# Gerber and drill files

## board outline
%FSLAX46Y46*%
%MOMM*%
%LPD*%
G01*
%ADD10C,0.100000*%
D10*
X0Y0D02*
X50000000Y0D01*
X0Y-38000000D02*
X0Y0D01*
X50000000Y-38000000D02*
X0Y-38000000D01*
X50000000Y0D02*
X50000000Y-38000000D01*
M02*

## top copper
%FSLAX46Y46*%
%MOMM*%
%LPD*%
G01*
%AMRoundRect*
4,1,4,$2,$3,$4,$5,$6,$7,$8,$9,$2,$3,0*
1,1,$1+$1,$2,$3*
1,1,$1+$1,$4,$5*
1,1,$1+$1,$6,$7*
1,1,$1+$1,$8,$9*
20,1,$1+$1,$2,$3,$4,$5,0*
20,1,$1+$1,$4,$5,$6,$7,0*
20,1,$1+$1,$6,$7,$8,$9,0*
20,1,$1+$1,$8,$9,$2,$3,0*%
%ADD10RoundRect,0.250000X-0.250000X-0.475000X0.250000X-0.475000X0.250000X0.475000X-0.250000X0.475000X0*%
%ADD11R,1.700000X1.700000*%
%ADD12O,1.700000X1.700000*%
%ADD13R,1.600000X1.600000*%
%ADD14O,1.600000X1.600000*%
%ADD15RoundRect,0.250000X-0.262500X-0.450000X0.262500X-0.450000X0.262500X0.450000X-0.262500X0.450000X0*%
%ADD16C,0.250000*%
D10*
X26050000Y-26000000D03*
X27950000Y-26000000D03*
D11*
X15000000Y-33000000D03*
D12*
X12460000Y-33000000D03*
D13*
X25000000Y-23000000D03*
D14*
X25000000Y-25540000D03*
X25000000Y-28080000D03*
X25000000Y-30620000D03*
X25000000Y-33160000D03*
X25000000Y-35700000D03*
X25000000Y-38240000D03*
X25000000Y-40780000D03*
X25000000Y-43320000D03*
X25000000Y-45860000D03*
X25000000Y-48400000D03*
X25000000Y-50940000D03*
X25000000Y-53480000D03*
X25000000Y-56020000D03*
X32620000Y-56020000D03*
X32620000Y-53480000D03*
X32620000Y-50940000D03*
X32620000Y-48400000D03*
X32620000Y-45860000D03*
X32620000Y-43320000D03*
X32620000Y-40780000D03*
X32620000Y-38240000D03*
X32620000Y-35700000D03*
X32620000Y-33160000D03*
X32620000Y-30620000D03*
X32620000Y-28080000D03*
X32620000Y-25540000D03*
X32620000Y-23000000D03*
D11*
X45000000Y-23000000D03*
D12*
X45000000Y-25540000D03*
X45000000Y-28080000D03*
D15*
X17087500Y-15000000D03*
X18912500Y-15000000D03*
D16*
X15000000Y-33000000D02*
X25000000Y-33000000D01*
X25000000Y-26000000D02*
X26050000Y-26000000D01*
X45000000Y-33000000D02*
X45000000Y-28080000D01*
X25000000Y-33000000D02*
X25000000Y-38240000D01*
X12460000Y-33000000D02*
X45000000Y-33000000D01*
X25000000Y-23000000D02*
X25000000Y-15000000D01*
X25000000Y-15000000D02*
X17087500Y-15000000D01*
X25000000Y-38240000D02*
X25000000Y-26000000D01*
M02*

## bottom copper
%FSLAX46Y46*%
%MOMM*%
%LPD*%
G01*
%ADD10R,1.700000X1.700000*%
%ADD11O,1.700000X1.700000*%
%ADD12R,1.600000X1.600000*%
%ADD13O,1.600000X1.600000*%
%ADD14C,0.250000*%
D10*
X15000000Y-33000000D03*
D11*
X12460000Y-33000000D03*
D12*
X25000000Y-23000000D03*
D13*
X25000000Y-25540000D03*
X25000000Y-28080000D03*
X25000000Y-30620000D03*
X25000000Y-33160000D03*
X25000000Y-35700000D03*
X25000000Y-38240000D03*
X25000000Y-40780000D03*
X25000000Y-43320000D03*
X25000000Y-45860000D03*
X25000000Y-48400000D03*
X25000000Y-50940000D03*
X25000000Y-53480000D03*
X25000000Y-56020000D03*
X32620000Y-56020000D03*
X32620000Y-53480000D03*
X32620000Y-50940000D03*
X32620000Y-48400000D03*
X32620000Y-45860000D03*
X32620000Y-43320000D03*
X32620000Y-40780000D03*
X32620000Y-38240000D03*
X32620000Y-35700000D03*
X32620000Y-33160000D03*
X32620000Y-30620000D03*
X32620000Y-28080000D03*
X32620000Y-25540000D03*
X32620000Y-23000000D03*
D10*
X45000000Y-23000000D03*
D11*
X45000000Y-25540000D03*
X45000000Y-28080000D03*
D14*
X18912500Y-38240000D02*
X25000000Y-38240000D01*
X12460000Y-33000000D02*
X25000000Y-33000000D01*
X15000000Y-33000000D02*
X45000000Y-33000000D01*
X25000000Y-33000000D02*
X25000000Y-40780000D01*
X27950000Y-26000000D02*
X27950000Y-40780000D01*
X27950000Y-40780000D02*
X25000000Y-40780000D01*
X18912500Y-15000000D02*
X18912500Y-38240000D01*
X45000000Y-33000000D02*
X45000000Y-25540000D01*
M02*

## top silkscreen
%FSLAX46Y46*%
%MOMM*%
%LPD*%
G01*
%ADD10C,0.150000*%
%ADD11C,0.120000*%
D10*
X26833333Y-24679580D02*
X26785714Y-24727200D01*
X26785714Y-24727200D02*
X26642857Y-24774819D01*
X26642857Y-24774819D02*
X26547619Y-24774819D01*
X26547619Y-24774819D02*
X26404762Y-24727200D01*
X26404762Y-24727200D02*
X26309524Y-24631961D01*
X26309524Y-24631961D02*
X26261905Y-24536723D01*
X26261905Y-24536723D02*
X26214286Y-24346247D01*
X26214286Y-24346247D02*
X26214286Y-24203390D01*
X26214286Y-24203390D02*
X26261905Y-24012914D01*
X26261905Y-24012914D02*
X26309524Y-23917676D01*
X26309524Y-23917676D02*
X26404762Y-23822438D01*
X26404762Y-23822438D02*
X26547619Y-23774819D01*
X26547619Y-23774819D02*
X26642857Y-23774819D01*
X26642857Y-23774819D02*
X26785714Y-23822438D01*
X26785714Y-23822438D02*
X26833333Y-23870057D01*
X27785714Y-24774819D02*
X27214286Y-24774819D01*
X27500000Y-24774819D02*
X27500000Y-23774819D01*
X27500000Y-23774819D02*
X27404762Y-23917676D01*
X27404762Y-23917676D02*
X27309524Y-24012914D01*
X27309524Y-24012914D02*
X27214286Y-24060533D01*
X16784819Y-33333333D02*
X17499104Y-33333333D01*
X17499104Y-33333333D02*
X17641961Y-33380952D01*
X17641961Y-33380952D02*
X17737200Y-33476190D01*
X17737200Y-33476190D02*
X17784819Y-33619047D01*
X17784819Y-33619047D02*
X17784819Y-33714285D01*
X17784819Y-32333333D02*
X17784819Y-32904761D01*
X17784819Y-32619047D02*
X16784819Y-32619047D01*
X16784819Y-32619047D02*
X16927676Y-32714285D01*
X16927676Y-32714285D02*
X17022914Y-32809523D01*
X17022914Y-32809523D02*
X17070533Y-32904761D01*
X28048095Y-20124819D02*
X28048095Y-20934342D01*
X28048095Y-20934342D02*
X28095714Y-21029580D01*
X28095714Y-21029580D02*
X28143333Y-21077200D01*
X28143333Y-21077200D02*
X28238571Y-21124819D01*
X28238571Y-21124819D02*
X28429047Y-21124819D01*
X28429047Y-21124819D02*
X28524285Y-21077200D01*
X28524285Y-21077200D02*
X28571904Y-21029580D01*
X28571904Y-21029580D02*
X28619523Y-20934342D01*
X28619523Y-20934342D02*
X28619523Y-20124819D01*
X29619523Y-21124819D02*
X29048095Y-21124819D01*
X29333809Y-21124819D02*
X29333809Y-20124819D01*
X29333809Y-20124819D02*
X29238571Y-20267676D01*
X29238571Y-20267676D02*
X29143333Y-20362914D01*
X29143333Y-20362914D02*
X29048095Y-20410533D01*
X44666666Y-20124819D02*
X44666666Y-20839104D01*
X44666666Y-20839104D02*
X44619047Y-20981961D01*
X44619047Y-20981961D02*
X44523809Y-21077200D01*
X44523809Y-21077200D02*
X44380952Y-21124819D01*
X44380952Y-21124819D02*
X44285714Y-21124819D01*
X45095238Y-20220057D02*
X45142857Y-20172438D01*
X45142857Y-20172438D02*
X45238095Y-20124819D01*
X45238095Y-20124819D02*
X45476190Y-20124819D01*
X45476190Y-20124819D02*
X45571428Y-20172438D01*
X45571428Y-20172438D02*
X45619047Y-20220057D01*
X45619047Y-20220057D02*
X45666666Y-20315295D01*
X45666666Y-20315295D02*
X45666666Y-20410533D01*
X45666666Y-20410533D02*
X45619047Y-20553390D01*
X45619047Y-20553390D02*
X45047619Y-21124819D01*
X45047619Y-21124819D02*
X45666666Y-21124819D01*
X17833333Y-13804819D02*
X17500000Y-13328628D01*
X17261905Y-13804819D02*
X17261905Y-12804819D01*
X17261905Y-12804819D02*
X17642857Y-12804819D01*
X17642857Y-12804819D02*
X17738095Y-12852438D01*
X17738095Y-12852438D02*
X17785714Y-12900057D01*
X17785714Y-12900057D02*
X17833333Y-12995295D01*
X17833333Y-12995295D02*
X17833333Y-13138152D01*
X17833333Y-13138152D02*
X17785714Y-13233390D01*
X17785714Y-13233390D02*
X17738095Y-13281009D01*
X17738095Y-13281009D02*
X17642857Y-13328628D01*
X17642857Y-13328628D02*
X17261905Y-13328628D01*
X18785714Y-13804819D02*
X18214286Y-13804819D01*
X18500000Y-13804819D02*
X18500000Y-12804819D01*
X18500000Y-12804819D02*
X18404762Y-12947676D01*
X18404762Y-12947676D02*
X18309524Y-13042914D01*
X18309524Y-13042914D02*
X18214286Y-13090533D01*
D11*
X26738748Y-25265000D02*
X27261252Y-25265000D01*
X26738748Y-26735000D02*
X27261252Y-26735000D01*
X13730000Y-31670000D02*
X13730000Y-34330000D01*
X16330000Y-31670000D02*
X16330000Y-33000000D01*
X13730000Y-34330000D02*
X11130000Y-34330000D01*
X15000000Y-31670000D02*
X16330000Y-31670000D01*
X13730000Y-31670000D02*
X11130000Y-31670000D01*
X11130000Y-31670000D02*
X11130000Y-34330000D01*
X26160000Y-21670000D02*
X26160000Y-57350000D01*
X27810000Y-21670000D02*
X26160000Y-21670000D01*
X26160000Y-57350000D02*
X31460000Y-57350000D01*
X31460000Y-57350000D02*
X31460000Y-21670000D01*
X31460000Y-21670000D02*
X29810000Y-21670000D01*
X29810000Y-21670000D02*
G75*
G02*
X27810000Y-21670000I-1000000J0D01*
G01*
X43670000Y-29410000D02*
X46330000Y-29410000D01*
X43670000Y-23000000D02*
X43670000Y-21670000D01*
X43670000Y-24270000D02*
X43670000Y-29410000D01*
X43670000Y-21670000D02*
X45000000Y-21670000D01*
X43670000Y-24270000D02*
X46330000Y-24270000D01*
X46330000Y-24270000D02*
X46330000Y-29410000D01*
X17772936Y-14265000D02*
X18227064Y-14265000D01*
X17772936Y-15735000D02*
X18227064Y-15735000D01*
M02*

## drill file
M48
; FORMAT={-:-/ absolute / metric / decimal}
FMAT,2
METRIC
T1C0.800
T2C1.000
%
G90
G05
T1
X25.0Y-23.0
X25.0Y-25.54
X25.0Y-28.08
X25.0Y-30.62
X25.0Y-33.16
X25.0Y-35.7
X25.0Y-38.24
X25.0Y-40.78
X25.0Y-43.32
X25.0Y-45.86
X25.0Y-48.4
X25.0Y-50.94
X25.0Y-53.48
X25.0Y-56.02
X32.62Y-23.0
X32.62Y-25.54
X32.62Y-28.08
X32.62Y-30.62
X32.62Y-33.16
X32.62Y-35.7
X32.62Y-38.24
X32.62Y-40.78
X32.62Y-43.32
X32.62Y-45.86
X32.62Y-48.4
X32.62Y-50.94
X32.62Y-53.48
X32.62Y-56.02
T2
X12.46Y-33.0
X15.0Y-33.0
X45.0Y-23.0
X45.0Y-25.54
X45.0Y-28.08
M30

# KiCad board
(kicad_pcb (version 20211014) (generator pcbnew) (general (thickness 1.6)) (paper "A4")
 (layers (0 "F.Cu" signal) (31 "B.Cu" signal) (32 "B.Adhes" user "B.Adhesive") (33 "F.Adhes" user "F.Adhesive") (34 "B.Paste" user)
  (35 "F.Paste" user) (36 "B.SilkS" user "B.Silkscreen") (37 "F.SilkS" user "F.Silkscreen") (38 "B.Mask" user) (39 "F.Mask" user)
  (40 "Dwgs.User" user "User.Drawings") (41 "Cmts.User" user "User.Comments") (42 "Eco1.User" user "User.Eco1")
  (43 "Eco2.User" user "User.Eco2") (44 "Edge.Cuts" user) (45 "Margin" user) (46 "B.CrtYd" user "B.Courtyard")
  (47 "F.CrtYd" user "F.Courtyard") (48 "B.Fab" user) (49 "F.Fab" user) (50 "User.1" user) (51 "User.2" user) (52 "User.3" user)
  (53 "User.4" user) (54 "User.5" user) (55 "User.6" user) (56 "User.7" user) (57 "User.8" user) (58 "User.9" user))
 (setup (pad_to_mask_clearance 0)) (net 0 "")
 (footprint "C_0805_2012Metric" (layer "F.Cu") (at 27 26)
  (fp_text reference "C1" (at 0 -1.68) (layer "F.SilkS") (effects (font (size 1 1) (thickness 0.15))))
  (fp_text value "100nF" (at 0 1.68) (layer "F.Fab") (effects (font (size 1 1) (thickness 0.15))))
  (fp_line (start -0.261252 -0.735) (end 0.261252 -0.735) (layer "F.SilkS") (width 0.12))
  (fp_line (start -0.261252 0.735) (end 0.261252 0.735) (layer "F.SilkS") (width 0.12))
  (pad "1" smd roundrect (at -0.95 0) (size 1 1.45) (layers "F.Cu" "F.Paste" "F.Mask") (roundrect_rratio 0.25))
  (pad "2" smd roundrect (at 0.95 0) (size 1 1.45) (layers "F.Cu" "F.Paste" "F.Mask") (roundrect_rratio 0.25)))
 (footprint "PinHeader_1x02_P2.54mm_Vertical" (layer "F.Cu") (at 15 33 -90)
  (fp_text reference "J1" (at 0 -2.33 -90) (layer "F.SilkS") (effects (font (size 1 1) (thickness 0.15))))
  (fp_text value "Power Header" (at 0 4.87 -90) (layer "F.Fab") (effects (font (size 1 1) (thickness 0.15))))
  (fp_line (start -1.33 1.27) (end 1.33 1.27) (layer "F.SilkS") (width 0.12))
  (fp_line (start -1.33 -1.33) (end 0 -1.33) (layer "F.SilkS") (width 0.12))
  (fp_line (start 1.33 1.27) (end 1.33 3.87) (layer "F.SilkS") (width 0.12))
  (fp_line (start -1.33 0) (end -1.33 -1.33) (layer "F.SilkS") (width 0.12))
  (fp_line (start -1.33 1.27) (end -1.33 3.87) (layer "F.SilkS") (width 0.12))
  (fp_line (start -1.33 3.87) (end 1.33 3.87) (layer "F.SilkS") (width 0.12))
  (pad "1" thru_hole rect (at 0 0 270) (size 1.7 1.7) (drill 1) (layers *.Cu *.Mask))
  (pad "2" thru_hole oval (at 0 2.54 270) (size 1.7 1.7) (drill 1) (layers *.Cu *.Mask)))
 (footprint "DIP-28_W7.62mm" (layer "F.Cu") (at 25 23)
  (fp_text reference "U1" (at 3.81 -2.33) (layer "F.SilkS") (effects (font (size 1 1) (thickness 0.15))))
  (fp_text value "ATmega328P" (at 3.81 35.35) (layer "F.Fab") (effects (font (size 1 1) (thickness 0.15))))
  (fp_line (start 1.16 -1.33) (end 1.16 34.35) (layer "F.SilkS") (width 0.12))
  (fp_line (start 2.81 -1.33) (end 1.16 -1.33) (layer "F.SilkS") (width 0.12))
  (fp_line (start 1.16 34.35) (end 6.46 34.35) (layer "F.SilkS") (width 0.12))
  (fp_line (start 6.46 34.35) (end 6.46 -1.33) (layer "F.SilkS") (width 0.12))
  (fp_line (start 6.46 -1.33) (end 4.81 -1.33) (layer "F.SilkS") (width 0.12))
  (fp_arc (start 4.81 -1.33) (mid 3.81 -0.33) (end 2.81 -1.33) (layer "F.SilkS") (width 0.12))
  (pad "1" thru_hole rect (at 0 0) (size 1.6 1.6) (drill 0.8) (layers *.Cu *.Mask))
  (pad "2" thru_hole oval (at 0 2.54) (size 1.6 1.6) (drill 0.8) (layers *.Cu *.Mask))
  (pad "3" thru_hole oval (at 0 5.08) (size 1.6 1.6) (drill 0.8) (layers *.Cu *.Mask))
  (pad "4" thru_hole oval (at 0 7.62) (size 1.6 1.6) (drill 0.8) (layers *.Cu *.Mask))
  (pad "5" thru_hole oval (at 0 10.16) (size 1.6 1.6) (drill 0.8) (layers *.Cu *.Mask))
  (pad "6" thru_hole oval (at 0 12.7) (size 1.6 1.6) (drill 0.8) (layers *.Cu *.Mask))
  (pad "7" thru_hole oval (at 0 15.24) (size 1.6 1.6) (drill 0.8) (layers *.Cu *.Mask))
  (pad "8" thru_hole oval (at 0 17.78) (size 1.6 1.6) (drill 0.8) (layers *.Cu *.Mask))
  (pad "9" thru_hole oval (at 0 20.32) (size 1.6 1.6) (drill 0.8) (layers *.Cu *.Mask))
  (pad "10" thru_hole oval (at 0 22.86) (size 1.6 1.6) (drill 0.8) (layers *.Cu *.Mask))
  (pad "11" thru_hole oval (at 0 25.4) (size 1.6 1.6) (drill 0.8) (layers *.Cu *.Mask))
  (pad "12" thru_hole oval (at 0 27.94) (size 1.6 1.6) (drill 0.8) (layers *.Cu *.Mask))
  (pad "13" thru_hole oval (at 0 30.48) (size 1.6 1.6) (drill 0.8) (layers *.Cu *.Mask))
  (pad "14" thru_hole oval (at 0 33.02) (size 1.6 1.6) (drill 0.8) (layers *.Cu *.Mask))
  (pad "15" thru_hole oval (at 7.62 33.02) (size 1.6 1.6) (drill 0.8) (layers *.Cu *.Mask))
  (pad "16" thru_hole oval (at 7.62 30.48) (size 1.6 1.6) (drill 0.8) (layers *.Cu *.Mask))
  (pad "17" thru_hole oval (at 7.62 27.94) (size 1.6 1.6) (drill 0.8) (layers *.Cu *.Mask))
  (pad "18" thru_hole oval (at 7.62 25.4) (size 1.6 1.6) (drill 0.8) (layers *.Cu *.Mask))
  (pad "19" thru_hole oval (at 7.62 22.86) (size 1.6 1.6) (drill 0.8) (layers *.Cu *.Mask))
  (pad "20" thru_hole oval (at 7.62 20.32) (size 1.6 1.6) (drill 0.8) (layers *.Cu *.Mask))
  (pad "21" thru_hole oval (at 7.62 17.78) (size 1.6 1.6) (drill 0.8) (layers *.Cu *.Mask))
  (pad "22" thru_hole oval (at 7.62 15.24) (size 1.6 1.6) (drill 0.8) (layers *.Cu *.Mask))
  (pad "23" thru_hole oval (at 7.62 12.7) (size 1.6 1.6) (drill 0.8) (layers *.Cu *.Mask))
  (pad "24" thru_hole oval (at 7.62 10.16) (size 1.6 1.6) (drill 0.8) (layers *.Cu *.Mask))
  (pad "25" thru_hole oval (at 7.62 7.62) (size 1.6 1.6) (drill 0.8) (layers *.Cu *.Mask))
  (pad "26" thru_hole oval (at 7.62 5.08) (size 1.6 1.6) (drill 0.8) (layers *.Cu *.Mask))
  (pad "27" thru_hole oval (at 7.62 2.54) (size 1.6 1.6) (drill 0.8) (layers *.Cu *.Mask))
  (pad "28" thru_hole oval (at 7.62 0) (size 1.6 1.6) (drill 0.8) (layers *.Cu *.Mask)))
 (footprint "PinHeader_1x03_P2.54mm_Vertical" (layer "F.Cu") (at 45 23)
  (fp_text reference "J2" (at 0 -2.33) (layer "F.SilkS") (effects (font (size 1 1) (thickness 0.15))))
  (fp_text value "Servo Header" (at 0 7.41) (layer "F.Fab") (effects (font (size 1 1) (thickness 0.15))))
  (fp_line (start -1.33 6.41) (end 1.33 6.41) (layer "F.SilkS") (width 0.12))
  (fp_line (start -1.33 0) (end -1.33 -1.33) (layer "F.SilkS") (width 0.12))
  (fp_line (start -1.33 1.27) (end -1.33 6.41) (layer "F.SilkS") (width 0.12))
  (fp_line (start -1.33 -1.33) (end 0 -1.33) (layer "F.SilkS") (width 0.12))
  (fp_line (start -1.33 1.27) (end 1.33 1.27) (layer "F.SilkS") (width 0.12))
  (fp_line (start 1.33 1.27) (end 1.33 6.41) (layer "F.SilkS") (width 0.12))
  (pad "1" thru_hole rect (at 0 0) (size 1.7 1.7) (drill 1) (layers *.Cu *.Mask))
  (pad "2" thru_hole oval (at 0 2.54) (size 1.7 1.7) (drill 1) (layers *.Cu *.Mask))
  (pad "3" thru_hole oval (at 0 5.08) (size 1.7 1.7) (drill 1) (layers *.Cu *.Mask)))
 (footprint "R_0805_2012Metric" (layer "F.Cu") (at 18 15)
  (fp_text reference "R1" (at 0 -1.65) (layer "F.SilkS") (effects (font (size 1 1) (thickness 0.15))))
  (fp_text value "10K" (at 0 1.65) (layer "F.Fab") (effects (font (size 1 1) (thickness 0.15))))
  (fp_line (start -0.227064 -0.735) (end 0.227064 -0.735) (layer "F.SilkS") (width 0.12))
  (fp_line (start -0.227064 0.735) (end 0.227064 0.735) (layer "F.SilkS") (width 0.12))
  (pad "1" smd roundrect (at -0.9125 0) (size 1.025 1.4) (layers "F.Cu" "F.Paste" "F.Mask") (roundrect_rratio 0.243902))
  (pad "2" smd roundrect (at 0.9125 0) (size 1.025 1.4) (layers "F.Cu" "F.Paste" "F.Mask") (roundrect_rratio 0.243902)))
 (gr_line (start 0 0) (end 50 0) (layer "Edge.Cuts") (width 0.1))
 (gr_line (start 0 38) (end 0 0) (layer "Edge.Cuts") (width 0.1))
 (gr_line (start 50 38) (end 0 38) (layer "Edge.Cuts") (width 0.1))
 (gr_line (start 50 0) (end 50 38) (layer "Edge.Cuts") (width 0.1))
 (segment (start 15 33) (end 25 33) (width 0.25) (layer "F.Cu") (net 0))
 (segment (start 25 26) (end 26.05 26) (width 0.25) (layer "F.Cu") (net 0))
 (segment (start 45 33) (end 45 28.08) (width 0.25) (layer "F.Cu") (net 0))
 (segment (start 25 33) (end 25 38.24) (width 0.25) (layer "F.Cu") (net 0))
 (segment (start 12.46 33) (end 45 33) (width 0.25) (layer "F.Cu") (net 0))
 (segment (start 25 23) (end 25 15) (width 0.25) (layer "F.Cu") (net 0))
 (segment (start 25 15) (end 17.0875 15) (width 0.25) (layer "F.Cu") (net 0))
 (segment (start 25 38.24) (end 25 26) (width 0.25) (layer "F.Cu") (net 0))
 (segment (start 18.9125 38.24) (end 25 38.24) (width 0.25) (layer "B.Cu") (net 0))
 (segment (start 12.46 33) (end 25 33) (width 0.25) (layer "B.Cu") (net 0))
 (segment (start 15 33) (end 45 33) (width 0.25) (layer "B.Cu") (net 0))
 (segment (start 25 33) (end 25 40.78) (width 0.25) (layer "B.Cu") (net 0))
 (segment (start 27.95 26) (end 27.95 40.78) (width 0.25) (layer "B.Cu") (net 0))
 (segment (start 27.95 40.78) (end 25 40.78) (width 0.25) (layer "B.Cu") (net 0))
 (segment (start 18.9125 15) (end 18.9125 38.24) (width 0.25) (layer "B.Cu") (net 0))
 (segment (start 45 33) (end 45 25.54) (width 0.25) (layer "B.Cu") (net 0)))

